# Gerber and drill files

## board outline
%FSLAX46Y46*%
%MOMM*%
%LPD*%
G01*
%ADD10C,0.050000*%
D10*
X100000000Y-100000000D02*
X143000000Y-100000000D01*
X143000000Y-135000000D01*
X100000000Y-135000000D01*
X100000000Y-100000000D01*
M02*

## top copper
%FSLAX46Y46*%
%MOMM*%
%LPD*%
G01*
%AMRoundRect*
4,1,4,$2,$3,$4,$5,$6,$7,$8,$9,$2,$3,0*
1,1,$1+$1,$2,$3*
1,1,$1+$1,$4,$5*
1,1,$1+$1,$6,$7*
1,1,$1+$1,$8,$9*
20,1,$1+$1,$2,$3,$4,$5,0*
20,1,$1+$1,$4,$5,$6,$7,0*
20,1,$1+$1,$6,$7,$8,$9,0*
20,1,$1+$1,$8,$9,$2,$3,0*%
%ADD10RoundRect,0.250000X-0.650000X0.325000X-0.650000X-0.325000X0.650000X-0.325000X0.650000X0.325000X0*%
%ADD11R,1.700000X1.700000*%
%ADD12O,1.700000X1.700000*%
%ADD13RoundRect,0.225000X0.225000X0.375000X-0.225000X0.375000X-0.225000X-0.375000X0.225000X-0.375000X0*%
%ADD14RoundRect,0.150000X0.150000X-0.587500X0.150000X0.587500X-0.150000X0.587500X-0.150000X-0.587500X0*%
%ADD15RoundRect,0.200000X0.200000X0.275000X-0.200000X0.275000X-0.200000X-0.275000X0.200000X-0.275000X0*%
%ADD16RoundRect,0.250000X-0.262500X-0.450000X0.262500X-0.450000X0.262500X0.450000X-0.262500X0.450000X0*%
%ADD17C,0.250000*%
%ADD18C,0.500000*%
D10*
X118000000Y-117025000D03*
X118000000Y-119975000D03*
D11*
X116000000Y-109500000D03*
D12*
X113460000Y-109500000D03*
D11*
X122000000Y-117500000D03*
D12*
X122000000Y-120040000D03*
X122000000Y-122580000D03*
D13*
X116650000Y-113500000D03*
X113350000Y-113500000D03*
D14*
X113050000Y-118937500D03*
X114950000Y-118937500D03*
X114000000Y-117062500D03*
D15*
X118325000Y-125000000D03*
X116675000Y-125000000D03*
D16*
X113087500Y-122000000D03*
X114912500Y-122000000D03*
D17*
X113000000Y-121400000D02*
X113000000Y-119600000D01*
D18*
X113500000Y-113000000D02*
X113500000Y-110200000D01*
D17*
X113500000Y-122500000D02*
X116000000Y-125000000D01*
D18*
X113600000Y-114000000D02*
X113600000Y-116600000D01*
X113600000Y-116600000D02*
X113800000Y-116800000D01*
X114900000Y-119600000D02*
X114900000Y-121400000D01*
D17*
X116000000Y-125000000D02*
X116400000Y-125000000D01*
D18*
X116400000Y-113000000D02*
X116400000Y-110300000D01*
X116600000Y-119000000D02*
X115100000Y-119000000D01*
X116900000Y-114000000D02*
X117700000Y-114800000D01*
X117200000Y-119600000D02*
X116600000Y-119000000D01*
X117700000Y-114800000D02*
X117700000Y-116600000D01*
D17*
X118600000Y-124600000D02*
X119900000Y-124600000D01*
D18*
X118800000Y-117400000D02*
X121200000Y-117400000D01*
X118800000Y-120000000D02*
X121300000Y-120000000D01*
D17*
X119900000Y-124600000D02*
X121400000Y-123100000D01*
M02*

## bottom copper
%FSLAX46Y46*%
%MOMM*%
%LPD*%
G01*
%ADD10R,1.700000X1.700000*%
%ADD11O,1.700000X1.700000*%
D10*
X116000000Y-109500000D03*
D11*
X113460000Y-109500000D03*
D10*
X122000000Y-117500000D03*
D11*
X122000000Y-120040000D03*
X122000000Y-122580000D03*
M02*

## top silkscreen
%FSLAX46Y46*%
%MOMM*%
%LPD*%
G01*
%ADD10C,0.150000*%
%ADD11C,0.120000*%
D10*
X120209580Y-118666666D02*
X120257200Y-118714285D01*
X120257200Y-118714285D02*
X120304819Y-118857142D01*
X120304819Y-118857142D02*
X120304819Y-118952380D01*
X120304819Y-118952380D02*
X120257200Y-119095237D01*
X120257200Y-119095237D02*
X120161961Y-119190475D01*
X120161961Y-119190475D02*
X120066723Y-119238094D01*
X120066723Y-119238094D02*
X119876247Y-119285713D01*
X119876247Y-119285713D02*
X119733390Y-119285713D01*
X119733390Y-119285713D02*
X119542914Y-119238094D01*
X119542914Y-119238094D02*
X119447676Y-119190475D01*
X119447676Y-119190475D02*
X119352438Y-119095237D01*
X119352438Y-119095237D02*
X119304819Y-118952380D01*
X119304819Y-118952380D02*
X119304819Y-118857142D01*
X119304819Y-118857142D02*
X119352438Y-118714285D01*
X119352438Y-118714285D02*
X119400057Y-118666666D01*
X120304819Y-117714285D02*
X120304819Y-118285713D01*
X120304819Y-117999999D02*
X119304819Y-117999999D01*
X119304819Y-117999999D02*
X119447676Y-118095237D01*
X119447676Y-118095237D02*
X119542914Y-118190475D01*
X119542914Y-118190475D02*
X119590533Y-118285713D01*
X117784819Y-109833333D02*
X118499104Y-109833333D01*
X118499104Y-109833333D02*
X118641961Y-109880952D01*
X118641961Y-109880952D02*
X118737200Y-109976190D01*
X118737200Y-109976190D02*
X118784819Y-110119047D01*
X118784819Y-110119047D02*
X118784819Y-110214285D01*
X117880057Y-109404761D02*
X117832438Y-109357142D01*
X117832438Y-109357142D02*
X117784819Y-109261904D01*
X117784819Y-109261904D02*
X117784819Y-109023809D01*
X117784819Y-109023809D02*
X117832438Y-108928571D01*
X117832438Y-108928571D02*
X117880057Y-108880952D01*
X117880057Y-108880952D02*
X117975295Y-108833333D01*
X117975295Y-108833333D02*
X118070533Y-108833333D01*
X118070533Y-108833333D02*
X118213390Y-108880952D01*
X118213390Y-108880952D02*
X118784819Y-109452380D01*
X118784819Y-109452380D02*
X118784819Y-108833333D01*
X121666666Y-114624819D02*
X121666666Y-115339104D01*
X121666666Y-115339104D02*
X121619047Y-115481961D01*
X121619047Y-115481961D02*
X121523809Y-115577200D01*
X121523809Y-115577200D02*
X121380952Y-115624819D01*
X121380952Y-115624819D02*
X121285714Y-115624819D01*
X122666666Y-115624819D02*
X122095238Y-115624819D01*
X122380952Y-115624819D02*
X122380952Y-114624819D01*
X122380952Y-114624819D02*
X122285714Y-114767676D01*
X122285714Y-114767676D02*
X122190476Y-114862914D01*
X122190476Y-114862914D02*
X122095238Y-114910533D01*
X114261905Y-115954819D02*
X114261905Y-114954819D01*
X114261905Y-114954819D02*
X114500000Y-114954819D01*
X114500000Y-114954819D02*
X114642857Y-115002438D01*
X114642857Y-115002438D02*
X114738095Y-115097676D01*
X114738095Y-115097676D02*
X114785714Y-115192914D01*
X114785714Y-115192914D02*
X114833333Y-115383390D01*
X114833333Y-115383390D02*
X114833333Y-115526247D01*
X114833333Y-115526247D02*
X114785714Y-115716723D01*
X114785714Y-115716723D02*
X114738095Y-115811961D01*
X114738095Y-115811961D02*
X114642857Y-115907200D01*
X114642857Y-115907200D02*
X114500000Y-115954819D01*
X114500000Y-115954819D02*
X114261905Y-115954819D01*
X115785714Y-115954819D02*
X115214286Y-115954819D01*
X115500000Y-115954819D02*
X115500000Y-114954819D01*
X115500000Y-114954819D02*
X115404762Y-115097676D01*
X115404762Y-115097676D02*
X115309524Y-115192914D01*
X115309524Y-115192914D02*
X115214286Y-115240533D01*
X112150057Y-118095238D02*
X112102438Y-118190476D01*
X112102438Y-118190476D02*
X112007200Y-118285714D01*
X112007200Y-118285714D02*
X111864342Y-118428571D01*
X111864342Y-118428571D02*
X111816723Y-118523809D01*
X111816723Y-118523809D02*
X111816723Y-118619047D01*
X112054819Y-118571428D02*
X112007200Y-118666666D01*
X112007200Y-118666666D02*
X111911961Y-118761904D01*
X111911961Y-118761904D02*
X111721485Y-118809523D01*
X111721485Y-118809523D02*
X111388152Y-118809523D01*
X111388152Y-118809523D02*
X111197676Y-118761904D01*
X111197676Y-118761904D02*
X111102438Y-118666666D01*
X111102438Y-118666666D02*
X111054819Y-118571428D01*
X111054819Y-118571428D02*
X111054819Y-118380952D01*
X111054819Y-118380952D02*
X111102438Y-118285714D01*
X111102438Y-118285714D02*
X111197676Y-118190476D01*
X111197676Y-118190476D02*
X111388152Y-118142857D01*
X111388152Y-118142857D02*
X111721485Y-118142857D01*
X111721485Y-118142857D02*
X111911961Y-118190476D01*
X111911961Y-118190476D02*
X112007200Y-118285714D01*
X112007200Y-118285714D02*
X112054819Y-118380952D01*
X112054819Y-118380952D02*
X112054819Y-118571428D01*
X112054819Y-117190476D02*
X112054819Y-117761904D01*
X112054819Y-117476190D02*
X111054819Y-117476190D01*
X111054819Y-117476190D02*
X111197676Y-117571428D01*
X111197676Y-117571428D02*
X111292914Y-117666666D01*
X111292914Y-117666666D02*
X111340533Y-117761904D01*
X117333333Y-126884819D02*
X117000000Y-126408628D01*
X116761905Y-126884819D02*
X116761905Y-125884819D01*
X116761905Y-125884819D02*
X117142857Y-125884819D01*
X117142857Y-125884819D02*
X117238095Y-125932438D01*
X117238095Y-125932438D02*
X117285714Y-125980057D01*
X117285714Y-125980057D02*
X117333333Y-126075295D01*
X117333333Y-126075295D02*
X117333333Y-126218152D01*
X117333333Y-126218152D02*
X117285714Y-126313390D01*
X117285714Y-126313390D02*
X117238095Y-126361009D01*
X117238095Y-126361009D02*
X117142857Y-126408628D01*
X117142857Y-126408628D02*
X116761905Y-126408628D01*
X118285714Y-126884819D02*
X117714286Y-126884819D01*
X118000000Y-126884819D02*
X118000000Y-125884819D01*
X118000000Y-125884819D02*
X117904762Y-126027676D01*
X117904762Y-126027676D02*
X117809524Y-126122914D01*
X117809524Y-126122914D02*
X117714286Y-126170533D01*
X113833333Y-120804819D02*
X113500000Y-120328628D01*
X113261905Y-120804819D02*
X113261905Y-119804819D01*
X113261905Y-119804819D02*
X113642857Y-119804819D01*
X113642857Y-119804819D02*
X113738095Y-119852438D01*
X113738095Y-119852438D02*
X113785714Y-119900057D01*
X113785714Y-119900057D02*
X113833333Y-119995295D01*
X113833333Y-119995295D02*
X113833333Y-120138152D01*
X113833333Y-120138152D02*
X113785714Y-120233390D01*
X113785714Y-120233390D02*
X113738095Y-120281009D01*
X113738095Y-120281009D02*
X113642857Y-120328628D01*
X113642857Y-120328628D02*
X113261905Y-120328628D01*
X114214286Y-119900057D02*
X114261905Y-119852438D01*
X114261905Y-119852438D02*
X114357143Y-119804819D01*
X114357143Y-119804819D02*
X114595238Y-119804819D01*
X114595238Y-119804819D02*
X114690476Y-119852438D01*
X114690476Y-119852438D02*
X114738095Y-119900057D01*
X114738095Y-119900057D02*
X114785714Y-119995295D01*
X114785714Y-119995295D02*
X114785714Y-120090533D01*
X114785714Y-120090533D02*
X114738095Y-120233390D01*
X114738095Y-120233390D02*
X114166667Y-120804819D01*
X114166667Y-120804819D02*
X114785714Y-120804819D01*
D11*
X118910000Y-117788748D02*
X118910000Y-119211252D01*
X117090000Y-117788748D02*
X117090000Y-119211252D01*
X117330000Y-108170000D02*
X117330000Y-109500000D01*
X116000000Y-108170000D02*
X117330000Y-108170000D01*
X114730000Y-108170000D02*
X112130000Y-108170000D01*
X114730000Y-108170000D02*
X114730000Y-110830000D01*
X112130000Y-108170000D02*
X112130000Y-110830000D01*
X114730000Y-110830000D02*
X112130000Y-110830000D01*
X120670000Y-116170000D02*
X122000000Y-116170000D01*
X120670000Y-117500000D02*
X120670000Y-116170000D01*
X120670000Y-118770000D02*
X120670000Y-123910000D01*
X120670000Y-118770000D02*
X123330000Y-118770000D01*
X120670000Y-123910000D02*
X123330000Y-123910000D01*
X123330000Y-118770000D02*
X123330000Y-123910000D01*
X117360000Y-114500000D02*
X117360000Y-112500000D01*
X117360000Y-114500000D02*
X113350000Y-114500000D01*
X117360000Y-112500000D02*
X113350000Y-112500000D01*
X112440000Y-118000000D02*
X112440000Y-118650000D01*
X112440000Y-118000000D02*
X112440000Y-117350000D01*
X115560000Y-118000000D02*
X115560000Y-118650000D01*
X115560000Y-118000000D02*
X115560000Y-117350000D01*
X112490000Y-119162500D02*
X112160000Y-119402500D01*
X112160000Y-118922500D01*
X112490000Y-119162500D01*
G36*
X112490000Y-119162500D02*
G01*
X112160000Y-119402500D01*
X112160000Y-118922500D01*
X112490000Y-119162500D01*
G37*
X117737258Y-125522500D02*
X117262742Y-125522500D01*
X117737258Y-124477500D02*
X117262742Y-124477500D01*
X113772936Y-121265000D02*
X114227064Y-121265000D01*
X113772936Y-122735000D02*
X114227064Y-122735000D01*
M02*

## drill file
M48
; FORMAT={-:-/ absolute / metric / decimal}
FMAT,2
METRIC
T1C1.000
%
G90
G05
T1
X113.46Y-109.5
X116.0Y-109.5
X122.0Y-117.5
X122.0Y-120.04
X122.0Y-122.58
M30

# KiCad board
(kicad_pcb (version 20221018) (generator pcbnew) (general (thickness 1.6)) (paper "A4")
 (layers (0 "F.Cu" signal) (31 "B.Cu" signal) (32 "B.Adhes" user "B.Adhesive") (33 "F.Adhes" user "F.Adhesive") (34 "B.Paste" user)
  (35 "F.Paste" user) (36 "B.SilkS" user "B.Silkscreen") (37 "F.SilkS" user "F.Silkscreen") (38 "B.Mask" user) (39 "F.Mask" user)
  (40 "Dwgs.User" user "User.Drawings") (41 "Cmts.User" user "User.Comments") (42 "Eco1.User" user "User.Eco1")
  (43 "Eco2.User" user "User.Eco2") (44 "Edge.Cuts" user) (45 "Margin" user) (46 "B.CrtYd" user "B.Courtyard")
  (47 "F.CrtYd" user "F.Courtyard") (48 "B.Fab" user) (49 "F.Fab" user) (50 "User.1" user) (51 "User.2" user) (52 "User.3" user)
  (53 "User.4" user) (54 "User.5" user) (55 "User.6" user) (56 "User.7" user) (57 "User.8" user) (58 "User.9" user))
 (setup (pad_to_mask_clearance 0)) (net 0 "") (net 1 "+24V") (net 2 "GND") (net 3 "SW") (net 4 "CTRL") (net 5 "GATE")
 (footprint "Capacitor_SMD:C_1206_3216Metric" (layer "F.Cu") (at 118 118.5 -90)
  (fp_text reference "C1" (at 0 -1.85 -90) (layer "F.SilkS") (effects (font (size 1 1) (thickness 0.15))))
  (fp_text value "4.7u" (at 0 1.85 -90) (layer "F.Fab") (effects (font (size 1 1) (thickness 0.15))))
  (fp_line (start -0.711252 -0.91) (end 0.711252 -0.91) (stroke (width 0.12) (type solid)) (layer "F.SilkS"))
  (fp_line (start -0.711252 0.91) (end 0.711252 0.91) (stroke (width 0.12) (type solid)) (layer "F.SilkS"))
  (pad "1" smd roundrect (at -1.475 0 270) (size 1.15 1.8) (layers "F.Cu" "F.Paste" "F.Mask") (roundrect_rratio 0.217391) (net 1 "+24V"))
  (pad "2" smd roundrect (at 1.475 0 270) (size 1.15 1.8) (layers "F.Cu" "F.Paste" "F.Mask") (roundrect_rratio 0.217391) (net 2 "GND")))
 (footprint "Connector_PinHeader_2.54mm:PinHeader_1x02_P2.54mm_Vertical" (layer "F.Cu") (at 116 109.5 -90)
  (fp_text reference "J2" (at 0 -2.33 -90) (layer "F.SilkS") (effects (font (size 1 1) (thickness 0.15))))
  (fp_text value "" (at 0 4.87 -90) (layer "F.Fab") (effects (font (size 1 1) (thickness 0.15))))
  (fp_line (start -1.33 -1.33) (end 0 -1.33) (stroke (width 0.12) (type solid)) (layer "F.SilkS"))
  (fp_line (start -1.33 0) (end -1.33 -1.33) (stroke (width 0.12) (type solid)) (layer "F.SilkS"))
  (fp_line (start -1.33 1.27) (end -1.33 3.87) (stroke (width 0.12) (type solid)) (layer "F.SilkS"))
  (fp_line (start -1.33 1.27) (end 1.33 1.27) (stroke (width 0.12) (type solid)) (layer "F.SilkS"))
  (fp_line (start -1.33 3.87) (end 1.33 3.87) (stroke (width 0.12) (type solid)) (layer "F.SilkS"))
  (fp_line (start 1.33 1.27) (end 1.33 3.87) (stroke (width 0.12) (type solid)) (layer "F.SilkS"))
  (pad "1" thru_hole rect (at 0 0 270) (size 1.7 1.7) (drill 1) (layers "*.Cu" "*.Mask") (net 1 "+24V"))
  (pad "2" thru_hole oval (at 0 2.54 270) (size 1.7 1.7) (drill 1) (layers "*.Cu" "*.Mask") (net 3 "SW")))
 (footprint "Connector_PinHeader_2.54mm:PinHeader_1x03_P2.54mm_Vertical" (layer "F.Cu") (at 122 117.5)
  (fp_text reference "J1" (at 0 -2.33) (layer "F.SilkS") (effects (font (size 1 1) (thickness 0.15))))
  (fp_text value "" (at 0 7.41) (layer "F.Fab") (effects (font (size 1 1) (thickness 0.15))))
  (fp_line (start -1.33 -1.33) (end 0 -1.33) (stroke (width 0.12) (type solid)) (layer "F.SilkS"))
  (fp_line (start -1.33 0) (end -1.33 -1.33) (stroke (width 0.12) (type solid)) (layer "F.SilkS"))
  (fp_line (start -1.33 1.27) (end -1.33 6.41) (stroke (width 0.12) (type solid)) (layer "F.SilkS"))
  (fp_line (start -1.33 1.27) (end 1.33 1.27) (stroke (width 0.12) (type solid)) (layer "F.SilkS"))
  (fp_line (start -1.33 6.41) (end 1.33 6.41) (stroke (width 0.12) (type solid)) (layer "F.SilkS"))
  (fp_line (start 1.33 1.27) (end 1.33 6.41) (stroke (width 0.12) (type solid)) (layer "F.SilkS"))
  (pad "1" thru_hole rect (at 0 0) (size 1.7 1.7) (drill 1) (layers "*.Cu" "*.Mask") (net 1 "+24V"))
  (pad "2" thru_hole oval (at 0 2.54) (size 1.7 1.7) (drill 1) (layers "*.Cu" "*.Mask") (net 2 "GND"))
  (pad "3" thru_hole oval (at 0 5.08) (size 1.7 1.7) (drill 1) (layers "*.Cu" "*.Mask") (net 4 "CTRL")))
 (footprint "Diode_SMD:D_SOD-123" (layer "F.Cu") (at 115 113.5 180)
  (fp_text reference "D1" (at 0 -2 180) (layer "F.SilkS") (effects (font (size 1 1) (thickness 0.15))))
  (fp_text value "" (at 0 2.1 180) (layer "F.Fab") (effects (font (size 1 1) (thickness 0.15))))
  (fp_line (start -2.36 -1) (end -2.36 1) (stroke (width 0.12) (type solid)) (layer "F.SilkS"))
  (fp_line (start -2.36 -1) (end 1.65 -1) (stroke (width 0.12) (type solid)) (layer "F.SilkS"))
  (fp_line (start -2.36 1) (end 1.65 1) (stroke (width 0.12) (type solid)) (layer "F.SilkS"))
  (pad "1" smd roundrect (at -1.65 0 180) (size 0.9 1.2) (layers "F.Cu" "F.Paste" "F.Mask") (roundrect_rratio 0.25) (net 1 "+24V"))
  (pad "2" smd roundrect (at 1.65 0 180) (size 0.9 1.2) (layers "F.Cu" "F.Paste" "F.Mask") (roundrect_rratio 0.25) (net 3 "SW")))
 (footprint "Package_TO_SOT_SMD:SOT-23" (layer "F.Cu") (at 114 118 90)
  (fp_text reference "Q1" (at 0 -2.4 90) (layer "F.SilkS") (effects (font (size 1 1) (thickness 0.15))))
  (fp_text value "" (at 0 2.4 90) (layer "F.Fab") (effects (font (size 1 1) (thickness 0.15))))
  (fp_line (start 0 -1.56) (end -0.65 -1.56) (stroke (width 0.12) (type solid)) (layer "F.SilkS"))
  (fp_line (start 0 -1.56) (end 0.65 -1.56) (stroke (width 0.12) (type solid)) (layer "F.SilkS"))
  (fp_line (start 0 1.56) (end -0.65 1.56) (stroke (width 0.12) (type solid)) (layer "F.SilkS"))
  (fp_line (start 0 1.56) (end 0.65 1.56) (stroke (width 0.12) (type solid)) (layer "F.SilkS"))
  (fp_poly
   (pts (xy -1.1625 -1.51) (xy -1.4025 -1.84) (xy -0.9225 -1.84) (xy -1.1625 -1.51)) (stroke (width 0.12) (type solid)) (fill solid)
   (layer "F.SilkS"))
  (pad "1" smd roundrect (at -0.9375 -0.95 90) (size 1.475 0.6) (layers "F.Cu" "F.Paste" "F.Mask") (roundrect_rratio 0.25) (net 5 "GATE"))
  (pad "2" smd roundrect (at -0.9375 0.95 90) (size 1.475 0.6) (layers "F.Cu" "F.Paste" "F.Mask") (roundrect_rratio 0.25) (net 2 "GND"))
  (pad "3" smd roundrect (at 0.9375 0 90) (size 1.475 0.6) (layers "F.Cu" "F.Paste" "F.Mask") (roundrect_rratio 0.25) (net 3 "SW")))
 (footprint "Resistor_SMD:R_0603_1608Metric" (layer "F.Cu") (at 117.5 125 180)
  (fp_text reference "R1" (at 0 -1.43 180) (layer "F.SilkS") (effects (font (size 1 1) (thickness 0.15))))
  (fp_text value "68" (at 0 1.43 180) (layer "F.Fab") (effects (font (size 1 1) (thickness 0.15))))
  (fp_line (start -0.237258 -0.5225) (end 0.237258 -0.5225) (stroke (width 0.12) (type solid)) (layer "F.SilkS"))
  (fp_line (start -0.237258 0.5225) (end 0.237258 0.5225) (stroke (width 0.12) (type solid)) (layer "F.SilkS"))
  (pad "1" smd roundrect (at -0.825 0 180) (size 0.8 0.95) (layers "F.Cu" "F.Paste" "F.Mask") (roundrect_rratio 0.25) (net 4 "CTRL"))
  (pad "2" smd roundrect (at 0.825 0 180) (size 0.8 0.95) (layers "F.Cu" "F.Paste" "F.Mask") (roundrect_rratio 0.25) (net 5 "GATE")))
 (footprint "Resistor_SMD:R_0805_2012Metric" (layer "F.Cu") (at 114 122)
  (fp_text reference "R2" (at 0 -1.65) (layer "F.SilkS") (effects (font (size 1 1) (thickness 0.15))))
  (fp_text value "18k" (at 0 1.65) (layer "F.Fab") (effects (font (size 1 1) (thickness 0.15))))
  (fp_line (start -0.227064 -0.735) (end 0.227064 -0.735) (stroke (width 0.12) (type solid)) (layer "F.SilkS"))
  (fp_line (start -0.227064 0.735) (end 0.227064 0.735) (stroke (width 0.12) (type solid)) (layer "F.SilkS"))
  (pad "1" smd roundrect (at -0.9125 0) (size 1.025 1.4) (layers "F.Cu" "F.Paste" "F.Mask") (roundrect_rratio 0.243902) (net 5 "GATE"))
  (pad "2" smd roundrect (at 0.9125 0) (size 1.025 1.4) (layers "F.Cu" "F.Paste" "F.Mask") (roundrect_rratio 0.243902) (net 2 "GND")))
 (gr_rect (start 100 100) (end 143 135) (stroke (width 0.05) (type default)) (fill none) (layer "Edge.Cuts"))
 (segment (start 113 121.4) (end 113 119.6) (width 0.25) (layer "F.Cu") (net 5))
 (segment (start 113.5 113) (end 113.5 110.2) (width 0.5) (layer "F.Cu") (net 3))
 (segment (start 113.5 122.5) (end 116 125) (width 0.25) (layer "F.Cu") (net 5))
 (segment (start 113.6 114) (end 113.6 116.6) (width 0.5) (layer "F.Cu") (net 3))
 (segment (start 113.6 116.6) (end 113.8 116.8) (width 0.5) (layer "F.Cu") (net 3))
 (segment (start 114.9 119.6) (end 114.9 121.4) (width 0.5) (layer "F.Cu") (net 2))
 (segment (start 116 125) (end 116.4 125) (width 0.25) (layer "F.Cu") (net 5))
 (segment (start 116.4 113) (end 116.4 110.3) (width 0.5) (layer "F.Cu") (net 1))
 (segment (start 116.6 119) (end 115.1 119) (width 0.5) (layer "F.Cu") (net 2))
 (segment (start 116.9 114) (end 117.7 114.8) (width 0.5) (layer "F.Cu") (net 1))
 (segment (start 117.2 119.6) (end 116.6 119) (width 0.5) (layer "F.Cu") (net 2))
 (segment (start 117.7 114.8) (end 117.7 116.6) (width 0.5) (layer "F.Cu") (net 1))
 (segment (start 118.6 124.6) (end 119.9 124.6) (width 0.25) (layer "F.Cu") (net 4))
 (segment (start 118.8 117.4) (end 121.2 117.4) (width 0.5) (layer "F.Cu") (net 1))
 (segment (start 118.8 120) (end 121.3 120) (width 0.5) (layer "F.Cu") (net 2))
 (segment (start 119.9 124.6) (end 121.4 123.1) (width 0.25) (layer "F.Cu") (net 4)))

